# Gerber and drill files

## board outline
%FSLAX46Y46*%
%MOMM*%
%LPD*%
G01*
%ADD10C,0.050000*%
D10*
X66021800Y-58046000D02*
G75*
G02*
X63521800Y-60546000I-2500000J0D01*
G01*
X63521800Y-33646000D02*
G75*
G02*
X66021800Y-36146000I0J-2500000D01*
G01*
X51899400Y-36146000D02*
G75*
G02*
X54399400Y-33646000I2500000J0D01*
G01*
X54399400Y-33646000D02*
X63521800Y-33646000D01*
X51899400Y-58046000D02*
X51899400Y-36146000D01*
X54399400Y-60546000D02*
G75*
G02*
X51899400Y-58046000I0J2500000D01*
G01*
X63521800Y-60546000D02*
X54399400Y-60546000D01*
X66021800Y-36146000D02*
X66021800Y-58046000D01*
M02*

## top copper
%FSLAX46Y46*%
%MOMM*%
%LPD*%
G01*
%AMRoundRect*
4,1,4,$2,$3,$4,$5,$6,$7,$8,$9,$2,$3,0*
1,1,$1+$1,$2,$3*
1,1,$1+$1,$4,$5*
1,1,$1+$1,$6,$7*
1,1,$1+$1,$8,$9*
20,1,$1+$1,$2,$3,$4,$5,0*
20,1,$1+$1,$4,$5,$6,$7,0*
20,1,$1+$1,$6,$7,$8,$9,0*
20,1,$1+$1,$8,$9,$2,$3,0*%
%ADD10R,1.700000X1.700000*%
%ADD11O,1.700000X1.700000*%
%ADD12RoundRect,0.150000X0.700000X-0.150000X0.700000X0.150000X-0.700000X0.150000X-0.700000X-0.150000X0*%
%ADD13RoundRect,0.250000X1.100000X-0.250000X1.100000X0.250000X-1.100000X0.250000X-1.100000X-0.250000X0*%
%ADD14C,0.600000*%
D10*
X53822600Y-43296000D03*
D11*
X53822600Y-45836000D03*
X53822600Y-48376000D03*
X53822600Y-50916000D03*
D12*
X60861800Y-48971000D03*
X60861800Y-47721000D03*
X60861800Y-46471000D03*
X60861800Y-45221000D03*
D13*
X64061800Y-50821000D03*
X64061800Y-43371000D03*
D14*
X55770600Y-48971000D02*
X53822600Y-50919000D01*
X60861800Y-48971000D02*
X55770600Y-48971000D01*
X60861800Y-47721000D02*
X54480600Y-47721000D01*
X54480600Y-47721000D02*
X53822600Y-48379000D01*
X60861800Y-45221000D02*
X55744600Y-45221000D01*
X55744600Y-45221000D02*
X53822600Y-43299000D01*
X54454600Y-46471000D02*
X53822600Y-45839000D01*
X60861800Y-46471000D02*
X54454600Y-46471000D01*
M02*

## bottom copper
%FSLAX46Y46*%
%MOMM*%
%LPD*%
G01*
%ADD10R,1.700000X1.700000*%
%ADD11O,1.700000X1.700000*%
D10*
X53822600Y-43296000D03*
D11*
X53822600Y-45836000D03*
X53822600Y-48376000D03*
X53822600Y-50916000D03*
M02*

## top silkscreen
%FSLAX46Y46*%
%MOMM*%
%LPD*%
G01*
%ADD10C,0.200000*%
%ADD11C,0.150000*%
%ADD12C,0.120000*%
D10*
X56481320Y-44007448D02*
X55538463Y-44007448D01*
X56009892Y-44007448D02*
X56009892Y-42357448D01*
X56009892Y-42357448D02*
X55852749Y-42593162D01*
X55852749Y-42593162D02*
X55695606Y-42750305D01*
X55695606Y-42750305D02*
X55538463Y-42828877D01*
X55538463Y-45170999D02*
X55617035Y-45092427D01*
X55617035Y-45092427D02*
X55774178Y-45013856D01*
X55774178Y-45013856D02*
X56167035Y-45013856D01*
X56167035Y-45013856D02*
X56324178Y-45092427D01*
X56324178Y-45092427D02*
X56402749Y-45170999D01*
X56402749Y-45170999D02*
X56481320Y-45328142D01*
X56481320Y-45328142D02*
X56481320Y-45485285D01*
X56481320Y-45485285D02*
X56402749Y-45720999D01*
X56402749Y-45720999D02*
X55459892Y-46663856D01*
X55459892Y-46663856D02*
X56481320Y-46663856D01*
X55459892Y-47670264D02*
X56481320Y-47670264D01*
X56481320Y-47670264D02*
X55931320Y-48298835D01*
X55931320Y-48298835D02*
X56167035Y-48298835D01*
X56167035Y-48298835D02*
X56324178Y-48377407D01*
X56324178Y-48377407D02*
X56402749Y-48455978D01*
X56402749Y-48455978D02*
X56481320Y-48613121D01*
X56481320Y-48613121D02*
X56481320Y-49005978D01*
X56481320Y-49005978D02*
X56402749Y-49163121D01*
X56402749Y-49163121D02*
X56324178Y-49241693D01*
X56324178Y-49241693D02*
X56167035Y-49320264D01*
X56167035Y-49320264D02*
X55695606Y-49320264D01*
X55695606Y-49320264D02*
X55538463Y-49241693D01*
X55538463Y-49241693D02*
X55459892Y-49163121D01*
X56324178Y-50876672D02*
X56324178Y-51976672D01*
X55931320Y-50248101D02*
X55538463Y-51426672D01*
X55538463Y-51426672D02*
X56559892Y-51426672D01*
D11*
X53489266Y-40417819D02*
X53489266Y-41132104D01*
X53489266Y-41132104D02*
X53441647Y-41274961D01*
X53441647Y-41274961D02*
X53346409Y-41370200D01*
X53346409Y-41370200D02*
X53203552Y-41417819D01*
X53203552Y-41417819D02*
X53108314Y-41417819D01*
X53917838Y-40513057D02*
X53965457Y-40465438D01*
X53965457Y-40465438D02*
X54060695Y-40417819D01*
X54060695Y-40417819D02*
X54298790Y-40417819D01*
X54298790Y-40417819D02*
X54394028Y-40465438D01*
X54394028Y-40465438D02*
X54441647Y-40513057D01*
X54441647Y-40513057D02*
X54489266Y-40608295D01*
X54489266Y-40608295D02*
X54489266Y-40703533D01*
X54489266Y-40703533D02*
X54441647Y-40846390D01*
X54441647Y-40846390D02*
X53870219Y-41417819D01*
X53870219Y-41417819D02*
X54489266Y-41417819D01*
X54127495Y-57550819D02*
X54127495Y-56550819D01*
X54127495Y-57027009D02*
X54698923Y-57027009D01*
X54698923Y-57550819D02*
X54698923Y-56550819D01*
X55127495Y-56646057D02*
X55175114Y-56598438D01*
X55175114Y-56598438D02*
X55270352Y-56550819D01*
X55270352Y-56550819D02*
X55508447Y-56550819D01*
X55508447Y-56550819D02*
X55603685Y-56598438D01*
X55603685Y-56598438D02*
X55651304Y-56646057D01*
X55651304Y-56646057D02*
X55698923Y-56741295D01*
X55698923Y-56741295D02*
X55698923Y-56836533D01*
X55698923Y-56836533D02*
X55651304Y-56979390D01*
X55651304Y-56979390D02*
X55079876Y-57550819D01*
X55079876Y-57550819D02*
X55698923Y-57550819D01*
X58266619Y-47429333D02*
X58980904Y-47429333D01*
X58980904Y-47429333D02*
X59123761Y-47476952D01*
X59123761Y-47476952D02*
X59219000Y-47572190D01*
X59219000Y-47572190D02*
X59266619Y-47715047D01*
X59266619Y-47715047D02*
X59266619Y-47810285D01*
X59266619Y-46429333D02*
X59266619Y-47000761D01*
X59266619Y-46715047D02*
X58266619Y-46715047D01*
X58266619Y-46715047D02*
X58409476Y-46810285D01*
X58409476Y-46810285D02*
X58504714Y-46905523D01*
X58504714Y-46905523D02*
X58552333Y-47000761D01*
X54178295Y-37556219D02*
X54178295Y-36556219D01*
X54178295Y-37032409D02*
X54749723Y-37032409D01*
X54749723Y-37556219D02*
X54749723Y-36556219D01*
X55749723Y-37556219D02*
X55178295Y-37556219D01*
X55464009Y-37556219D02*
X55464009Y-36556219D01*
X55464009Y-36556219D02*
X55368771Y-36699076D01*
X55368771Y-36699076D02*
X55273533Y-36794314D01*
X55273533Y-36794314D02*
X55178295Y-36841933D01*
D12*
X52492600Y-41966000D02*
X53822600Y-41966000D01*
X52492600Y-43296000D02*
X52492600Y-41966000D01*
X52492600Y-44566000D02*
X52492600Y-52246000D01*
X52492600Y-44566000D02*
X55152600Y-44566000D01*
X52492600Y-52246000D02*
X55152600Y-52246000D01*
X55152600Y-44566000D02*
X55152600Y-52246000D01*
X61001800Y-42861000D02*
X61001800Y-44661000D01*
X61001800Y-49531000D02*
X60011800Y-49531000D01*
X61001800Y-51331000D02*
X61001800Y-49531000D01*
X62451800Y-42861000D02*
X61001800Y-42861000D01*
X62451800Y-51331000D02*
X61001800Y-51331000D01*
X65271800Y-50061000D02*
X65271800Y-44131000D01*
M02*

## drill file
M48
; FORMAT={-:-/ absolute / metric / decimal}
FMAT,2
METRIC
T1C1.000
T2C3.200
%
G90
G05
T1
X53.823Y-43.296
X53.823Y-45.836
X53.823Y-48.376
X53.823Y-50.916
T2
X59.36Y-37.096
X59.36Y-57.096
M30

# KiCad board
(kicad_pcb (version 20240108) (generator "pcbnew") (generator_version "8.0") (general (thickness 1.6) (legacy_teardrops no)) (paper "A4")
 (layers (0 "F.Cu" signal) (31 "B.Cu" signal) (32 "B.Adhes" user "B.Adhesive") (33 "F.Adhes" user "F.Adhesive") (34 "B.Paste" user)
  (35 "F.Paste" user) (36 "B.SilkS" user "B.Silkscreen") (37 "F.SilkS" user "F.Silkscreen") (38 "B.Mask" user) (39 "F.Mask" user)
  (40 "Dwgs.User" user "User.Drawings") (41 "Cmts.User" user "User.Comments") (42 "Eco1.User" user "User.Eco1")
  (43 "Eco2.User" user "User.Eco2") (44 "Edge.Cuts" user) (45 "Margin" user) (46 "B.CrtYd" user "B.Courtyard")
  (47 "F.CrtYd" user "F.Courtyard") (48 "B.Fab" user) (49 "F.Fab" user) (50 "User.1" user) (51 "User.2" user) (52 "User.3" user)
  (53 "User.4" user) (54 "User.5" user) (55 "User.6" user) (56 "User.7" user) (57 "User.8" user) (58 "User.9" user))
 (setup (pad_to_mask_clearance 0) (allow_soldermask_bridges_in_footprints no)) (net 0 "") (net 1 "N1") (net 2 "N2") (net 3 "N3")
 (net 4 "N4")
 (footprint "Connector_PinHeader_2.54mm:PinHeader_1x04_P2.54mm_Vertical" (layer "F.Cu") (at 53.8226 43.296)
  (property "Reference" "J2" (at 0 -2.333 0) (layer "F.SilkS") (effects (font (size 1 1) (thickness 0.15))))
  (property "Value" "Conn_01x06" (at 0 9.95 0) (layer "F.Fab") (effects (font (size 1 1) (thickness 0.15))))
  (fp_line (start -1.33 -1.33) (end 0 -1.33) (stroke (width 0.12) (type solid)) (layer "F.SilkS"))
  (fp_line (start -1.33 0) (end -1.33 -1.33) (stroke (width 0.12) (type solid)) (layer "F.SilkS"))
  (fp_line (start -1.33 1.27) (end -1.33 8.95) (stroke (width 0.12) (type solid)) (layer "F.SilkS"))
  (fp_line (start -1.33 1.27) (end 1.33 1.27) (stroke (width 0.12) (type solid)) (layer "F.SilkS"))
  (fp_line (start -1.33 8.95) (end 1.33 8.95) (stroke (width 0.12) (type solid)) (layer "F.SilkS"))
  (fp_line (start 1.33 1.27) (end 1.33 8.95) (stroke (width 0.12) (type solid)) (layer "F.SilkS"))
  (pad "1" thru_hole rect (at 0 0) (size 1.7 1.7) (drill 1) (layers "*.Cu" "*.Mask") (remove_unused_layers no) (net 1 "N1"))
  (pad "2" thru_hole oval (at 0 2.54) (size 1.7 1.7) (drill 1) (layers "*.Cu" "*.Mask") (remove_unused_layers no) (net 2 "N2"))
  (pad "3" thru_hole oval (at 0 5.08) (size 1.7 1.7) (drill 1) (layers "*.Cu" "*.Mask") (remove_unused_layers no) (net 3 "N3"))
  (pad "4" thru_hole oval (at 0 7.62) (size 1.7 1.7) (drill 1) (layers "*.Cu" "*.Mask") (remove_unused_layers no) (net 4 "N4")))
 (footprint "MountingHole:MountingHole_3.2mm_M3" (layer "F.Cu") (at 59.3598 57.096)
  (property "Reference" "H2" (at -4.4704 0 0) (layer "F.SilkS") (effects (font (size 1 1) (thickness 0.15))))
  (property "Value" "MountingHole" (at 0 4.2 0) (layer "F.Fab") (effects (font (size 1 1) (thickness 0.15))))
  (pad "" np_thru_hole circle (at 0 0) (size 3.2 3.2) (drill 3.2) (layers "*.Cu" "*.Mask")))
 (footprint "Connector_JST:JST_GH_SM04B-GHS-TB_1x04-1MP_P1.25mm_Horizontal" (layer "F.Cu") (at 62.7118 47.096 90)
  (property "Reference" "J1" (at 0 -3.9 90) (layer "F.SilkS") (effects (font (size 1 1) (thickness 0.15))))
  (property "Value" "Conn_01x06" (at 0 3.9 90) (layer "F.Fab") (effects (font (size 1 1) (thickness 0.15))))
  (fp_line (start 4.235 -1.71) (end 2.435 -1.71) (stroke (width 0.12) (type solid)) (layer "F.SilkS"))
  (fp_line (start -2.435 -1.71) (end -2.435 -2.7) (stroke (width 0.12) (type solid)) (layer "F.SilkS"))
  (fp_line (start -4.235 -1.71) (end -2.435 -1.71) (stroke (width 0.12) (type solid)) (layer "F.SilkS"))
  (fp_line (start 4.235 -0.26) (end 4.235 -1.71) (stroke (width 0.12) (type solid)) (layer "F.SilkS"))
  (fp_line (start -4.235 -0.26) (end -4.235 -1.71) (stroke (width 0.12) (type solid)) (layer "F.SilkS"))
  (fp_line (start -2.965 2.56) (end 2.965 2.56) (stroke (width 0.12) (type solid)) (layer "F.SilkS"))
  (pad "1" smd roundrect (at -1.875 -1.85 90) (size 0.6 1.7) (layers "F.Cu" "F.Paste" "F.Mask") (roundrect_rratio 0.25) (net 4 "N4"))
  (pad "2" smd roundrect (at -0.625 -1.85 90) (size 0.6 1.7) (layers "F.Cu" "F.Paste" "F.Mask") (roundrect_rratio 0.25) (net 3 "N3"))
  (pad "3" smd roundrect (at 0.625 -1.85 90) (size 0.6 1.7) (layers "F.Cu" "F.Paste" "F.Mask") (roundrect_rratio 0.25) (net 2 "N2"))
  (pad "4" smd roundrect (at 1.875 -1.85 90) (size 0.6 1.7) (layers "F.Cu" "F.Paste" "F.Mask") (roundrect_rratio 0.25) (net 1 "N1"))
  (pad "MP" smd roundrect (at -3.725 1.35 90) (size 1 2.7) (layers "F.Cu" "F.Paste" "F.Mask") (roundrect_rratio 0.25))
  (pad "MP" smd roundrect (at 3.725 1.35 90) (size 1 2.7) (layers "F.Cu" "F.Paste" "F.Mask") (roundrect_rratio 0.25)))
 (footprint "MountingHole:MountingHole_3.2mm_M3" (layer "F.Cu") (at 59.3598 37.096)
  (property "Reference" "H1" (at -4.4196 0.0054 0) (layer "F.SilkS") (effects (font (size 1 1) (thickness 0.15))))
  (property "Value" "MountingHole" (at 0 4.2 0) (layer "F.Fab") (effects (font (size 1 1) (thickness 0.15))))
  (pad "" np_thru_hole circle (at 0 0) (size 3.2 3.2) (drill 3.2) (layers "*.Cu" "*.Mask")))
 (gr_arc (start 66.0218 58.046) (mid 65.289567 59.813767) (end 63.5218 60.546) (stroke (width 0.05) (type default)) (layer "Edge.Cuts"))
 (gr_arc (start 63.5218 33.646) (mid 65.289567 34.378233) (end 66.0218 36.146) (stroke (width 0.05) (type default)) (layer "Edge.Cuts"))
 (gr_arc (start 51.8994 36.146) (mid 52.631633 34.378233) (end 54.3994 33.646) (stroke (width 0.05) (type default)) (layer "Edge.Cuts"))
 (gr_line (start 54.3994 33.646) (end 63.5218 33.646) (stroke (width 0.05) (type default)) (layer "Edge.Cuts"))
 (gr_line (start 51.8994 58.046) (end 51.8994 36.146) (stroke (width 0.05) (type default)) (layer "Edge.Cuts"))
 (gr_arc (start 54.3994 60.546) (mid 52.631633 59.813767) (end 51.8994 58.046) (stroke (width 0.05) (type default)) (layer "Edge.Cuts"))
 (gr_line (start 63.5218 60.546) (end 54.3994 60.546) (stroke (width 0.05) (type default)) (layer "Edge.Cuts"))
 (gr_line (start 66.0218 36.146) (end 66.0218 58.046) (stroke (width 0.05) (type default)) (layer "Edge.Cuts"))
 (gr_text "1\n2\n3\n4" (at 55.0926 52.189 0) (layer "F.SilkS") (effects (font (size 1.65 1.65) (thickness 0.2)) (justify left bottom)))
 (segment (start 55.7706 48.971) (end 53.8226 50.919) (width 0.6) (layer "F.Cu") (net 4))
 (segment (start 60.8618 48.971) (end 55.7706 48.971) (width 0.6) (layer "F.Cu") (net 4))
 (segment (start 60.8618 47.721) (end 54.4806 47.721) (width 0.6) (layer "F.Cu") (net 3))
 (segment (start 54.4806 47.721) (end 53.8226 48.379) (width 0.6) (layer "F.Cu") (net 3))
 (segment (start 60.8618 45.221) (end 55.7446 45.221) (width 0.6) (layer "F.Cu") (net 1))
 (segment (start 55.7446 45.221) (end 53.8226 43.299) (width 0.6) (layer "F.Cu") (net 1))
 (segment (start 54.4546 46.471) (end 53.8226 45.839) (width 0.6) (layer "F.Cu") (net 2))
 (segment (start 60.8618 46.471) (end 54.4546 46.471) (width 0.6) (layer "F.Cu") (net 2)))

